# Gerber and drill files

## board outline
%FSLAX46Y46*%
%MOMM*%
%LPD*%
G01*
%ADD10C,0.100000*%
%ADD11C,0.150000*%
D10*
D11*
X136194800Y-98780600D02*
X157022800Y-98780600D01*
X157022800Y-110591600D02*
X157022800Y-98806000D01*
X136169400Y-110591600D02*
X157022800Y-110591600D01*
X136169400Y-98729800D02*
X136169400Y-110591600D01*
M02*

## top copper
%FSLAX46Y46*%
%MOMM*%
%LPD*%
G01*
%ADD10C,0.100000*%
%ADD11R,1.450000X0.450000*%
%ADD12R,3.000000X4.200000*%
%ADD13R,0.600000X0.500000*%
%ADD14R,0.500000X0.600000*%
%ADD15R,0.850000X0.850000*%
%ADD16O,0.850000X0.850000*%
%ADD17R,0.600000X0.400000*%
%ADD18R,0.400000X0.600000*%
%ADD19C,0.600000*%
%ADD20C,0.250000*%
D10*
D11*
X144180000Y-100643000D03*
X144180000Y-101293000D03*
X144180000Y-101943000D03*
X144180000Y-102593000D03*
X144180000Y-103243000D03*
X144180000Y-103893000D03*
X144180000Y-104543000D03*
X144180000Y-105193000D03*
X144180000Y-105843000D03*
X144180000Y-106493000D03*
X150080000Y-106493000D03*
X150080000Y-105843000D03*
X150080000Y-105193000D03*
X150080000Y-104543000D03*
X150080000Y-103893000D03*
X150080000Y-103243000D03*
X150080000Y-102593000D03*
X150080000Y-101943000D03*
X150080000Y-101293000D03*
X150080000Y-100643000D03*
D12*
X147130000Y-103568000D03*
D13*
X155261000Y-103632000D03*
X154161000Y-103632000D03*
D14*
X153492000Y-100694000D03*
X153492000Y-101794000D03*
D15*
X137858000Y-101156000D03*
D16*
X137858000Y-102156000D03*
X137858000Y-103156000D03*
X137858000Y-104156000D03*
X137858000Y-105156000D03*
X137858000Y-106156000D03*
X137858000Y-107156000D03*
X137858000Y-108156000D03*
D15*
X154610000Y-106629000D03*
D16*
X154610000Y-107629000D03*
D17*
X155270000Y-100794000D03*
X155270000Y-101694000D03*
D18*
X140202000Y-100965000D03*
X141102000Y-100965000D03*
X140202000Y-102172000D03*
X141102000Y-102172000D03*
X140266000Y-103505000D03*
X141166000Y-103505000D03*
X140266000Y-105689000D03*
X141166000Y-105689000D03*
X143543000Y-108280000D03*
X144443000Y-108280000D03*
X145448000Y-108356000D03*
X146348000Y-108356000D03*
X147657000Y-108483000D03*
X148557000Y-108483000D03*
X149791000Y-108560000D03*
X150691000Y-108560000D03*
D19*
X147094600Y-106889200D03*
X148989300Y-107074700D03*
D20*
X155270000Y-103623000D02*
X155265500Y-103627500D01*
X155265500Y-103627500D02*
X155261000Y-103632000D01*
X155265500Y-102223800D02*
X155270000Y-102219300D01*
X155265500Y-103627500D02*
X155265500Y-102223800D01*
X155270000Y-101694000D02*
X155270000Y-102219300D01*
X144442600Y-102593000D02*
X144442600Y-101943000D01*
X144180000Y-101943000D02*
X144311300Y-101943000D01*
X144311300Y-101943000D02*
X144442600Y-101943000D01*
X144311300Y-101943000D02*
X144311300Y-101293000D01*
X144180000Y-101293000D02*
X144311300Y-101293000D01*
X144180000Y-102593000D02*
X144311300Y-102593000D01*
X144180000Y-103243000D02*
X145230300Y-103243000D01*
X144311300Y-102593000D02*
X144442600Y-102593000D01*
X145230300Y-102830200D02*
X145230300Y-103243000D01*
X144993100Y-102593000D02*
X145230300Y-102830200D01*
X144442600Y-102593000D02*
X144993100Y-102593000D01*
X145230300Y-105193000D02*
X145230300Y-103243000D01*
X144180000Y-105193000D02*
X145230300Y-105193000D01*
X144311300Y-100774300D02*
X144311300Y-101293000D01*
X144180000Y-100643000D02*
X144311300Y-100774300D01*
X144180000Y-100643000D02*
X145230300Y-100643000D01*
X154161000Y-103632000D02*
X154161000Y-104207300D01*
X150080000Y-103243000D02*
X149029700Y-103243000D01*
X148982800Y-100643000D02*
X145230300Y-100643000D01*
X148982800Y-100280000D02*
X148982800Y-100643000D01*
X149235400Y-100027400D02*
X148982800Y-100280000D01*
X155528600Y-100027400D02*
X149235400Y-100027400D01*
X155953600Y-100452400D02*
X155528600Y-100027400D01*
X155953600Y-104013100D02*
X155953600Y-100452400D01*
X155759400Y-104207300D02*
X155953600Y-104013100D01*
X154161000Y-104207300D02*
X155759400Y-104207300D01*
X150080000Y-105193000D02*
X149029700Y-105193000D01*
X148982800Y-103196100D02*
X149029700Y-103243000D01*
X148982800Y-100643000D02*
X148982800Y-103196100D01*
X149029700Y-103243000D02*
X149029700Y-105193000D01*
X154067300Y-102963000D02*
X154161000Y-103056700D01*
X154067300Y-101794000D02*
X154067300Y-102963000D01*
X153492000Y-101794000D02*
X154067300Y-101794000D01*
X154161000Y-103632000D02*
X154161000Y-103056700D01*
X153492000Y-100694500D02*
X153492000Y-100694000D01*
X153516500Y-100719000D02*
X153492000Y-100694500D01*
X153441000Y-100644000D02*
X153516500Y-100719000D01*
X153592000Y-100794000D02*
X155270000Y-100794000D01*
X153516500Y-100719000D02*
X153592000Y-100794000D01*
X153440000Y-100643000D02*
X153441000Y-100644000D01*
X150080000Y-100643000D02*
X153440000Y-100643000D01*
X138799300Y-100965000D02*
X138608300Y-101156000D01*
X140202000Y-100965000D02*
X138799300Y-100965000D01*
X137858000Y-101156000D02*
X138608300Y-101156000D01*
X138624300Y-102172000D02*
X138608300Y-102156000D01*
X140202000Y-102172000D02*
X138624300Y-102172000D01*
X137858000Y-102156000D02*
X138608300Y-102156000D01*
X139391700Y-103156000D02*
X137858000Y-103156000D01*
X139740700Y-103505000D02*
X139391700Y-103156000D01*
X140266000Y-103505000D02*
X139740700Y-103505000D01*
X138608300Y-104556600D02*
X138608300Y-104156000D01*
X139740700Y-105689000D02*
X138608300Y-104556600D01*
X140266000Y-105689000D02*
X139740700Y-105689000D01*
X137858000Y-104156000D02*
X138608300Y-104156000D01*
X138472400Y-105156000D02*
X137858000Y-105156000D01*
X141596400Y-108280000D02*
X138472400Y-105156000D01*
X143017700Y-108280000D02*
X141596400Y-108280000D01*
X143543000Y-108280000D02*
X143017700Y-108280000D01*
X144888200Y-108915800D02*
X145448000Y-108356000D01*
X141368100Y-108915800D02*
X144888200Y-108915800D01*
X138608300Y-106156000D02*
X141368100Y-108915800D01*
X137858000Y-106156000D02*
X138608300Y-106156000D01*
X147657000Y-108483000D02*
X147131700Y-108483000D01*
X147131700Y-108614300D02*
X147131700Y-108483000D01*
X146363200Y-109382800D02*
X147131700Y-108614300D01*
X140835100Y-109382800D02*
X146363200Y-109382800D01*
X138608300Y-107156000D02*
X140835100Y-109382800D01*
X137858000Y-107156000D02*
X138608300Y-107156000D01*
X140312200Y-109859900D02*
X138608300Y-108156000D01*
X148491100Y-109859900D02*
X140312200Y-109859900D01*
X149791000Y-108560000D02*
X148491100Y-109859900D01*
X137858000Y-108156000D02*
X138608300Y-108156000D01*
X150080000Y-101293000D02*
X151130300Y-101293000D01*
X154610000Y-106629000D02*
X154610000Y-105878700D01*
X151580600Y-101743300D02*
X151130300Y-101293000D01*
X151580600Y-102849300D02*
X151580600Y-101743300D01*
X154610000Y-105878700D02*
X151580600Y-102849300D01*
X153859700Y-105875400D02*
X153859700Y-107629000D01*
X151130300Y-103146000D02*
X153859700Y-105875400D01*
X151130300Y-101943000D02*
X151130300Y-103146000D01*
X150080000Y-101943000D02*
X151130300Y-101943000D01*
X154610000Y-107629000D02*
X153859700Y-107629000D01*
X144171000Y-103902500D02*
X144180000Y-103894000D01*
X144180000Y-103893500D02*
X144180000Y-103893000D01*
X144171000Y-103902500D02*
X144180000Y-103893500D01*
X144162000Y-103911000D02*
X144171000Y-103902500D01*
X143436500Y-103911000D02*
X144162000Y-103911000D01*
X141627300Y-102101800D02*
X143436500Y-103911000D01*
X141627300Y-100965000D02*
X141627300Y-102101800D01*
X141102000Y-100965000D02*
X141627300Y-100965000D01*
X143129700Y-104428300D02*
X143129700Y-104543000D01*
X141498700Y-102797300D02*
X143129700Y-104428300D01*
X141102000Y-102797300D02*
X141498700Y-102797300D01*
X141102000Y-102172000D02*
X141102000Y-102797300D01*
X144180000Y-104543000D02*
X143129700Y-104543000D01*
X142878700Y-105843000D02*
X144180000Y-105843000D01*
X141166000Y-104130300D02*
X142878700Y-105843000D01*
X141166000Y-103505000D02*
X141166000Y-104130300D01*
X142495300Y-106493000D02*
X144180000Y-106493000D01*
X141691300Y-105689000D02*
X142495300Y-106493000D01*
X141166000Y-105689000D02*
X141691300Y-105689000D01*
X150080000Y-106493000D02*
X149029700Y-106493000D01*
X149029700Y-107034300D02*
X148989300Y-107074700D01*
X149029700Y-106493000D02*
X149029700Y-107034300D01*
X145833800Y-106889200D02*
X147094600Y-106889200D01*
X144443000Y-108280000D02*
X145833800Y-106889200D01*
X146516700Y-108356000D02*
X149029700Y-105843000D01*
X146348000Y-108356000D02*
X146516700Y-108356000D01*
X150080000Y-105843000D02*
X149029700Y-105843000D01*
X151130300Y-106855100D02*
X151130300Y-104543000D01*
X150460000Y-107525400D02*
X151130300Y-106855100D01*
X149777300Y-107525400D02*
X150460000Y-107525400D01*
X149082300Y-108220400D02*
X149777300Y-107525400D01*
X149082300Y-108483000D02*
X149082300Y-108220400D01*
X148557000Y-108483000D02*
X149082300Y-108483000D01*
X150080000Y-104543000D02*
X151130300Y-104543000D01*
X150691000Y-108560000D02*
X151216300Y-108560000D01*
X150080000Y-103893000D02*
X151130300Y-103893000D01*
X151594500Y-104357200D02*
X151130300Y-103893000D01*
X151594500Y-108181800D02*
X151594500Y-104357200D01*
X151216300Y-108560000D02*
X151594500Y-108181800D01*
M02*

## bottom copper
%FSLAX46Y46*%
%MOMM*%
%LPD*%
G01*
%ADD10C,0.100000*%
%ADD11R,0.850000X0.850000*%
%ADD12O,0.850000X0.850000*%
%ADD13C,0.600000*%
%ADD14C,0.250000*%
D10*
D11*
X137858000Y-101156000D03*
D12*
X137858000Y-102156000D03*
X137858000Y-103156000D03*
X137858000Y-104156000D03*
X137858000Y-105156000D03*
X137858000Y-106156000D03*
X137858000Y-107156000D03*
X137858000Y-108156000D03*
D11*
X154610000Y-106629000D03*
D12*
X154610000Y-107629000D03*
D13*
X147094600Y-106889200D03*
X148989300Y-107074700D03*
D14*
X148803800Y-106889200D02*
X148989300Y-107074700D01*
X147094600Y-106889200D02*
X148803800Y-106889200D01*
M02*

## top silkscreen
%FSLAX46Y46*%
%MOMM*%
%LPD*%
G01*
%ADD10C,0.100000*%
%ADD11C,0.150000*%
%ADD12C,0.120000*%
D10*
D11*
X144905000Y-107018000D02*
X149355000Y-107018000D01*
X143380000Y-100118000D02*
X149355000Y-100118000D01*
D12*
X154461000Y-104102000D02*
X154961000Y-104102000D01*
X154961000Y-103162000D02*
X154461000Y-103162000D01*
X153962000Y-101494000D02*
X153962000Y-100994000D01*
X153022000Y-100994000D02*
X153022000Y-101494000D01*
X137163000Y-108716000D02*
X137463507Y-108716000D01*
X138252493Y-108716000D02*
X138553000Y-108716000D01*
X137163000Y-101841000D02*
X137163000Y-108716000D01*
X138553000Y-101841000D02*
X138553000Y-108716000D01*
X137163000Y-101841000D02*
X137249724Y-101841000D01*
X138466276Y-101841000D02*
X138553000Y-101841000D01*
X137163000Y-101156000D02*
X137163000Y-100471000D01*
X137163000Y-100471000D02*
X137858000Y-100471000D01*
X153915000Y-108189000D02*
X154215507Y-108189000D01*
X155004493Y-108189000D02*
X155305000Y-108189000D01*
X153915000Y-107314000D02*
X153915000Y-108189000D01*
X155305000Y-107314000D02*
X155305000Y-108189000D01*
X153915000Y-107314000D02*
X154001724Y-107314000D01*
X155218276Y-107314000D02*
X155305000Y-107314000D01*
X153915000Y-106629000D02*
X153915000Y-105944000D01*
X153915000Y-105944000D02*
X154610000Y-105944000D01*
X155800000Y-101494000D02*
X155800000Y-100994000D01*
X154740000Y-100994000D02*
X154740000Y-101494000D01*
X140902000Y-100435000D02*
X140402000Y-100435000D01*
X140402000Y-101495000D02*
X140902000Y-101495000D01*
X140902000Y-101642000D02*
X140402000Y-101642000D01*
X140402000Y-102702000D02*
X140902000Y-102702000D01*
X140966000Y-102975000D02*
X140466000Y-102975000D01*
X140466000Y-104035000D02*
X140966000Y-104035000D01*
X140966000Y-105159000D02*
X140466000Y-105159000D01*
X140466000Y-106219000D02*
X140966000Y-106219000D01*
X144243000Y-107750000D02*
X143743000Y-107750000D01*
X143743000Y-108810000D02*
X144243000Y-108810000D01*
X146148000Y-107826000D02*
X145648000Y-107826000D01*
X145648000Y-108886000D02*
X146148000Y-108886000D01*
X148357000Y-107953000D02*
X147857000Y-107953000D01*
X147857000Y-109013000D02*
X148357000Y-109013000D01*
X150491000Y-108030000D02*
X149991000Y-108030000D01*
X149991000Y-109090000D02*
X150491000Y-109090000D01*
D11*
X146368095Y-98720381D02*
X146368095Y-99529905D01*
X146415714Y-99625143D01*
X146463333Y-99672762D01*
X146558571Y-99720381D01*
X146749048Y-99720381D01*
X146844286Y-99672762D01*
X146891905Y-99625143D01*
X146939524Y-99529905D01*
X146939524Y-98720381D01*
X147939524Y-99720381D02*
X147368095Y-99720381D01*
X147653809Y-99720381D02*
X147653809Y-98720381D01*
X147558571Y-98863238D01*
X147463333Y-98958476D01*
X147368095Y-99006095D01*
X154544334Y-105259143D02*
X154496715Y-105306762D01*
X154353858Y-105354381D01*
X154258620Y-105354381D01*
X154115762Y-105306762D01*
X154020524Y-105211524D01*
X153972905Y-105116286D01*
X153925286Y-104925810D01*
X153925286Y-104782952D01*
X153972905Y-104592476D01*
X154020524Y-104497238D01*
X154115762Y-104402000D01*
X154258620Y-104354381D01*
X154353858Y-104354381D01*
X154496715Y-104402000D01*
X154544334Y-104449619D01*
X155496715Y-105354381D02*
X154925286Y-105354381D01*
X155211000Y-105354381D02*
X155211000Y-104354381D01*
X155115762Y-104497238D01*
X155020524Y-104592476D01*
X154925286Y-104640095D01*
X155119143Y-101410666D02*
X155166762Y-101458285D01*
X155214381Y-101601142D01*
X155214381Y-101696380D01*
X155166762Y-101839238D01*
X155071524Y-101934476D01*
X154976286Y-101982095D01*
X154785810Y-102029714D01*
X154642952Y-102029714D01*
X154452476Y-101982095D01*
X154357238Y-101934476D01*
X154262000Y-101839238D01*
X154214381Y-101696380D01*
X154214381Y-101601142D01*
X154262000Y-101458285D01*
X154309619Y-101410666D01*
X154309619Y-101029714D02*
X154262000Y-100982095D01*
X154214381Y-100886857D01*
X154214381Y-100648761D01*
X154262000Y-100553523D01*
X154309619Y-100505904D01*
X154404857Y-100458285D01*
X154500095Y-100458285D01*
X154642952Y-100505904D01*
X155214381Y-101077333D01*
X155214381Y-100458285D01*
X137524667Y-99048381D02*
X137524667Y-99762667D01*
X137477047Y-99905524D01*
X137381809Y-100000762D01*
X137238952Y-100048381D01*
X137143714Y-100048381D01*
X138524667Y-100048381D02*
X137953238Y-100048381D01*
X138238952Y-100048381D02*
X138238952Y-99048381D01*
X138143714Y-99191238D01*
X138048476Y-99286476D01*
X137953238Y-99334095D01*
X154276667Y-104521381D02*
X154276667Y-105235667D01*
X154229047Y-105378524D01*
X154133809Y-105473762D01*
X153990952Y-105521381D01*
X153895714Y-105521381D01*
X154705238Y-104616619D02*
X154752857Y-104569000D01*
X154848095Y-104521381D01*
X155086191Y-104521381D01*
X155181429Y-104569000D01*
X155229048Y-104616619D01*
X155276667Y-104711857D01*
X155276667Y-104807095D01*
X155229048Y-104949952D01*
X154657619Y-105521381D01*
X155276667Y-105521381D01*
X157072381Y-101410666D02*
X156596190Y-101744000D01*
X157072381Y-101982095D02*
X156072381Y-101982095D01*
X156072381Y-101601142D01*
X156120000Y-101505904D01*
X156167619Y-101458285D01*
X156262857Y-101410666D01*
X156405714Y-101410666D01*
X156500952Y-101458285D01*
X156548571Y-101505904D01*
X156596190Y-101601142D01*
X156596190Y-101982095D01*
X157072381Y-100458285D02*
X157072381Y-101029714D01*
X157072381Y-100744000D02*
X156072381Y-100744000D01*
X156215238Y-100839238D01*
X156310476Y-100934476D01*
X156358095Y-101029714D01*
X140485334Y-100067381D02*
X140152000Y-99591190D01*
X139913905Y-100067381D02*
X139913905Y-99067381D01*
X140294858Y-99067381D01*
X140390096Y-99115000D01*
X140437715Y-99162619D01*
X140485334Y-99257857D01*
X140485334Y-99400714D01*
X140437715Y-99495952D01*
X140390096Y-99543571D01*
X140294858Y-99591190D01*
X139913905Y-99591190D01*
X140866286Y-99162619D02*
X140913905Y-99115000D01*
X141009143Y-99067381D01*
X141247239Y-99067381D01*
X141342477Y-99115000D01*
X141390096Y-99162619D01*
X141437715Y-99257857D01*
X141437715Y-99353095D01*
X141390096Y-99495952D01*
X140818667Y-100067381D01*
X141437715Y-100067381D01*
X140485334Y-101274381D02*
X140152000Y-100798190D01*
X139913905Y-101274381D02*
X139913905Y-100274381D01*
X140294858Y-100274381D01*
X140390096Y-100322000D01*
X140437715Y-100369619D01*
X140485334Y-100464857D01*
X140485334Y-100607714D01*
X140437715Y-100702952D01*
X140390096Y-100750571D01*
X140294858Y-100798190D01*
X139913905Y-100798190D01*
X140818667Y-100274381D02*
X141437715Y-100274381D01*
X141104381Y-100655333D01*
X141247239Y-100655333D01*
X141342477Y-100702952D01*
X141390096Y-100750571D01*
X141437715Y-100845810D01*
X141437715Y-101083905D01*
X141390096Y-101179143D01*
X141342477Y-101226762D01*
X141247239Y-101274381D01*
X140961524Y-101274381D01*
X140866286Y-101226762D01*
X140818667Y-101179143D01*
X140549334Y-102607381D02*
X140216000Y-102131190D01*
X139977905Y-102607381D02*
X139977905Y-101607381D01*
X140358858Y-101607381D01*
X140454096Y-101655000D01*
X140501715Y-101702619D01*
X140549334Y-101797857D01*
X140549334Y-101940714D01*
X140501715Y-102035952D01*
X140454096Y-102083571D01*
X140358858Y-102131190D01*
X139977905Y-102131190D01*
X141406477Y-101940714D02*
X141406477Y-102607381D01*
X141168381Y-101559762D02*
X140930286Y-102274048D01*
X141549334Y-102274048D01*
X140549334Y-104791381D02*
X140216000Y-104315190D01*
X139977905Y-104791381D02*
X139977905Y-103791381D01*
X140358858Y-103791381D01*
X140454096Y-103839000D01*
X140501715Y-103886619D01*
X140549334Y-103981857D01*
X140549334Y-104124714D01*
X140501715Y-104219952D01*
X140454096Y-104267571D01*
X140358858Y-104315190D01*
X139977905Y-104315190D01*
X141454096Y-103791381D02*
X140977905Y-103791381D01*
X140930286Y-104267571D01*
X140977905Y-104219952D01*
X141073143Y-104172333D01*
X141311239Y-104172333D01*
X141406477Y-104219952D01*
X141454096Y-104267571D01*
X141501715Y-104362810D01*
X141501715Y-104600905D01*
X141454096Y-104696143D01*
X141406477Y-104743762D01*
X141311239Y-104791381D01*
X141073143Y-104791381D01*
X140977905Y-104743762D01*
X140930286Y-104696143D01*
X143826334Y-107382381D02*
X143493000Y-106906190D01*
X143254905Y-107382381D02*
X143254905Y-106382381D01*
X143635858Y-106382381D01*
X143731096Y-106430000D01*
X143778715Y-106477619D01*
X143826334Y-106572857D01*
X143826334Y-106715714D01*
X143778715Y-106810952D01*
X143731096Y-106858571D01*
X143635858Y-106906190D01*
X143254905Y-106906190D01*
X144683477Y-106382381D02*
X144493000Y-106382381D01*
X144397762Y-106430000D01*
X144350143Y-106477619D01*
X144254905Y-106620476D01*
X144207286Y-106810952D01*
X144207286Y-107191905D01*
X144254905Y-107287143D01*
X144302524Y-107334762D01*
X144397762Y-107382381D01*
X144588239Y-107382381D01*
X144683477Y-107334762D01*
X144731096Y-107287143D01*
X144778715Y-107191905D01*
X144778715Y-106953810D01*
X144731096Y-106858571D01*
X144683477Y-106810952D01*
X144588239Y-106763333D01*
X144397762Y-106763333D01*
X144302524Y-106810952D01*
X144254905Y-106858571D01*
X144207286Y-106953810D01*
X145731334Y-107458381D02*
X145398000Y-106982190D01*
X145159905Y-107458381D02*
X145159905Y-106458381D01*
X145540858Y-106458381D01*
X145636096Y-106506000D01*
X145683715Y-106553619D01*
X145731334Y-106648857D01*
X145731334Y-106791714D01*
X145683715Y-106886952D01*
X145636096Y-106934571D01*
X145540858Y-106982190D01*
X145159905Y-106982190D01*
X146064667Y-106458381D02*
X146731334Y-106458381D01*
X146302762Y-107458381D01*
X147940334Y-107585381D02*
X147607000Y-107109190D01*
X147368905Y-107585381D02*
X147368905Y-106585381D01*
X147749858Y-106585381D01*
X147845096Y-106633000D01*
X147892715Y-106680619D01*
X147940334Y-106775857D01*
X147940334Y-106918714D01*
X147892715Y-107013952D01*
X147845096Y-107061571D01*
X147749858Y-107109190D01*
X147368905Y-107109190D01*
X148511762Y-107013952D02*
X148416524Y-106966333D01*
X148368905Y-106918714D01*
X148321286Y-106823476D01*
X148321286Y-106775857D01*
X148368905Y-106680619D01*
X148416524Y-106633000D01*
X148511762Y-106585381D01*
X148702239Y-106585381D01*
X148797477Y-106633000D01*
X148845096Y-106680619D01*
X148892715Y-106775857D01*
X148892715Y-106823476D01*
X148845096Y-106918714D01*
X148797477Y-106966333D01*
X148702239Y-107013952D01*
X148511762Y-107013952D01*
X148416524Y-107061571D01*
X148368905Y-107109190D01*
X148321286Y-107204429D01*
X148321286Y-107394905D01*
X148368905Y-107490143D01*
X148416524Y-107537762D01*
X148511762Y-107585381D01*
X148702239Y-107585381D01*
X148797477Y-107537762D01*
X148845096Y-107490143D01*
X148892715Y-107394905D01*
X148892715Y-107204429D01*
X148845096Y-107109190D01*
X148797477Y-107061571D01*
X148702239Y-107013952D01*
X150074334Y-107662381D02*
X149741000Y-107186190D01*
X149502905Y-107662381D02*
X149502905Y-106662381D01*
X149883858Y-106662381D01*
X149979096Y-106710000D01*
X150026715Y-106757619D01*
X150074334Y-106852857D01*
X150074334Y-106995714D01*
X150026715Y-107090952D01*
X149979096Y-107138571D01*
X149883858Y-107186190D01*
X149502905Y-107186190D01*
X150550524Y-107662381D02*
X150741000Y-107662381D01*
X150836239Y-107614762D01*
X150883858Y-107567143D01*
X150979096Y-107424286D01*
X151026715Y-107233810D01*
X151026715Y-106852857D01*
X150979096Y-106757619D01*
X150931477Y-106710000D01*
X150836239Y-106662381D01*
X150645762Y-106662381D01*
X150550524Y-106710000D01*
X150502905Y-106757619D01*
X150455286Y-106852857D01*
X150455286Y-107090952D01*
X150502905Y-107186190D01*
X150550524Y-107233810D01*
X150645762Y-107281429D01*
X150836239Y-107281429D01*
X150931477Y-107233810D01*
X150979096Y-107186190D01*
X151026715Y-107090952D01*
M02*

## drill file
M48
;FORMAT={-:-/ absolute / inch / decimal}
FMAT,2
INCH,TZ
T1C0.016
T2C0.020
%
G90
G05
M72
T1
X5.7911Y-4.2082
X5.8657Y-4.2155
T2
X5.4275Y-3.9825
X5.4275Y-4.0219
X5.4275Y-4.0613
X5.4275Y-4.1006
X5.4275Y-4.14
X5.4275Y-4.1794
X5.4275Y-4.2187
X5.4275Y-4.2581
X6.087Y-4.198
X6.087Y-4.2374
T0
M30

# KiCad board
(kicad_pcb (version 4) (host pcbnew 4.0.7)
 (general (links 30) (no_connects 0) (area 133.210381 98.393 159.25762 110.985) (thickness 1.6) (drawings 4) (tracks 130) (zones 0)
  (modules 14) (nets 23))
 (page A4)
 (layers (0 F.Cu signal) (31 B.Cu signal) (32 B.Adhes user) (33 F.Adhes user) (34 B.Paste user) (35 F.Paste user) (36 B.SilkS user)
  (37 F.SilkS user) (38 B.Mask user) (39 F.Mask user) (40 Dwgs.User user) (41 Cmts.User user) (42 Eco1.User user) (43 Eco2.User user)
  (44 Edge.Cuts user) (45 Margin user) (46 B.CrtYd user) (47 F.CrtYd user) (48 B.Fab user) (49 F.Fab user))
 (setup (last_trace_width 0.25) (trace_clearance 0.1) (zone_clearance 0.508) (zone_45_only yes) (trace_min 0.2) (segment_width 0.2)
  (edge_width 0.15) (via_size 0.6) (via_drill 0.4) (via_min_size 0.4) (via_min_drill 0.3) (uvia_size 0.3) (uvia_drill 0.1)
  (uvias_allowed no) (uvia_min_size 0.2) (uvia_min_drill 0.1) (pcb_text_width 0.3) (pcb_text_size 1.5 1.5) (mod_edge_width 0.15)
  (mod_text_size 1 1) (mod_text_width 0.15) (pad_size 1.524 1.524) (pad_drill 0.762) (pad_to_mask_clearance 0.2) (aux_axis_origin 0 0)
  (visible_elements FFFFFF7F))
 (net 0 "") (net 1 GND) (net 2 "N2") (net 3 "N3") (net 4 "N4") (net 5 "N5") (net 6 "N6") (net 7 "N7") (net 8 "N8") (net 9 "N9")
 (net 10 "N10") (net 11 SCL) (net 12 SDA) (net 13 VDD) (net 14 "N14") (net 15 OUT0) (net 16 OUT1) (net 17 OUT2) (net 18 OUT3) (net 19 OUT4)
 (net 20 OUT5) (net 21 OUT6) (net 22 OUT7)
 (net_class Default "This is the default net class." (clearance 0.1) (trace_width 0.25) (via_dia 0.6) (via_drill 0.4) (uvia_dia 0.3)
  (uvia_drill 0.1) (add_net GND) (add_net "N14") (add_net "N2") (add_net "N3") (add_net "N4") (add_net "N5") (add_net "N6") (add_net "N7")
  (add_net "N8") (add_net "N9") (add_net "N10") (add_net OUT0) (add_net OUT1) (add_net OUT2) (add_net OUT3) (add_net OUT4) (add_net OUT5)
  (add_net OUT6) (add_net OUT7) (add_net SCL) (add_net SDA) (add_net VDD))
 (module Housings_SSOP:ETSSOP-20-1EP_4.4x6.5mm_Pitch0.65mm (layer F.Cu) (at 147.13 103.568)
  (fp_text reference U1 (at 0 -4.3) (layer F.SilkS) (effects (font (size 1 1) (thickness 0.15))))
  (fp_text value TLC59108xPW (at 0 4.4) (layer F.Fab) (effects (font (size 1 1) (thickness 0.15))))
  (fp_line (start -2.225 3.45) (end 2.225 3.45) (layer F.SilkS) (width 0.15))
  (fp_line (start -3.75 -3.45) (end 2.225 -3.45) (layer F.SilkS) (width 0.15))
  (pad 1 smd rect (at -2.95 -2.925) (size 1.45 0.45) (layers F.Cu F.Paste F.Mask) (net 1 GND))
  (pad 2 smd rect (at -2.95 -2.275) (size 1.45 0.45) (layers F.Cu F.Paste F.Mask) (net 1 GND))
  (pad 3 smd rect (at -2.95 -1.625) (size 1.45 0.45) (layers F.Cu F.Paste F.Mask) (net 1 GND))
  (pad 4 smd rect (at -2.95 -0.975) (size 1.45 0.45) (layers F.Cu F.Paste F.Mask) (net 1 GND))
  (pad 5 smd rect (at -2.95 -0.325) (size 1.45 0.45) (layers F.Cu F.Paste F.Mask) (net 1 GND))
  (pad 6 smd rect (at -2.95 0.325) (size 1.45 0.45) (layers F.Cu F.Paste F.Mask) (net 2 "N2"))
  (pad 7 smd rect (at -2.95 0.975) (size 1.45 0.45) (layers F.Cu F.Paste F.Mask) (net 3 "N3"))
  (pad 8 smd rect (at -2.95 1.625) (size 1.45 0.45) (layers F.Cu F.Paste F.Mask) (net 1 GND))
  (pad 9 smd rect (at -2.95 2.275) (size 1.45 0.45) (layers F.Cu F.Paste F.Mask) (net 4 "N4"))
  (pad 10 smd rect (at -2.95 2.925) (size 1.45 0.45) (layers F.Cu F.Paste F.Mask) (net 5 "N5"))
  (pad 11 smd rect (at 2.95 2.925) (size 1.45 0.45) (layers F.Cu F.Paste F.Mask) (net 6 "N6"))
  (pad 12 smd rect (at 2.95 2.275) (size 1.45 0.45) (layers F.Cu F.Paste F.Mask) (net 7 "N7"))
  (pad 13 smd rect (at 2.95 1.625) (size 1.45 0.45) (layers F.Cu F.Paste F.Mask) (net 1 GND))
  (pad 14 smd rect (at 2.95 0.975) (size 1.45 0.45) (layers F.Cu F.Paste F.Mask) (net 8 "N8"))
  (pad 15 smd rect (at 2.95 0.325) (size 1.45 0.45) (layers F.Cu F.Paste F.Mask) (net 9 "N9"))
  (pad 16 smd rect (at 2.95 -0.325) (size 1.45 0.45) (layers F.Cu F.Paste F.Mask) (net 1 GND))
  (pad 17 smd rect (at 2.95 -0.975) (size 1.45 0.45) (layers F.Cu F.Paste F.Mask) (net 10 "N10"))
  (pad 18 smd rect (at 2.95 -1.625) (size 1.45 0.45) (layers F.Cu F.Paste F.Mask) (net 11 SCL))
  (pad 19 smd rect (at 2.95 -2.275) (size 1.45 0.45) (layers F.Cu F.Paste F.Mask) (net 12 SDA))
  (pad 20 smd rect (at 2.95 -2.925) (size 1.45 0.45) (layers F.Cu F.Paste F.Mask) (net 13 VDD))
  (pad 21 smd rect (at 0 0) (size 3 4.2) (layers F.Cu F.Paste F.Mask)))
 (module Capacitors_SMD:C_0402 (layer F.Cu) (at 154.711 103.632 180)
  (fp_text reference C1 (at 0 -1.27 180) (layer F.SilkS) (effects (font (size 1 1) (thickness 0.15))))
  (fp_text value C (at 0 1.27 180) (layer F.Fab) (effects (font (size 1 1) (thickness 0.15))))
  (fp_line (start 0.25 -0.47) (end -0.25 -0.47) (layer F.SilkS) (width 0.12))
  (fp_line (start -0.25 0.47) (end 0.25 0.47) (layer F.SilkS) (width 0.12))
  (pad 1 smd rect (at -0.55 0 180) (size 0.6 0.5) (layers F.Cu F.Paste F.Mask) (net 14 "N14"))
  (pad 2 smd rect (at 0.55 0 180) (size 0.6 0.5) (layers F.Cu F.Paste F.Mask) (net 1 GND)))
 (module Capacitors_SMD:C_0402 (layer F.Cu) (at 153.492 101.244 270)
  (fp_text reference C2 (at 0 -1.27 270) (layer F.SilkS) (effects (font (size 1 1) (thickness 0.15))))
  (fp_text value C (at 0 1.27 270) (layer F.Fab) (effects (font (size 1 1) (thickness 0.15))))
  (fp_line (start 0.25 -0.47) (end -0.25 -0.47) (layer F.SilkS) (width 0.12))
  (fp_line (start -0.25 0.47) (end 0.25 0.47) (layer F.SilkS) (width 0.12))
  (pad 1 smd rect (at -0.55 0 270) (size 0.6 0.5) (layers F.Cu F.Paste F.Mask) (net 13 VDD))
  (pad 2 smd rect (at 0.55 0 270) (size 0.6 0.5) (layers F.Cu F.Paste F.Mask) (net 1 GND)))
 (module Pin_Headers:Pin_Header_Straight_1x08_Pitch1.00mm (layer F.Cu) (at 137.858 101.156)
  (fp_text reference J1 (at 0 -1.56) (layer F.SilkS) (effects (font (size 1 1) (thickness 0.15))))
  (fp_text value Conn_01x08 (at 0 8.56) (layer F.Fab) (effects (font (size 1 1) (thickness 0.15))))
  (fp_line (start -0.695 7.56) (end -0.394493 7.56) (layer F.SilkS) (width 0.12))
  (fp_line (start 0.394493 7.56) (end 0.695 7.56) (layer F.SilkS) (width 0.12))
  (fp_line (start -0.695 0.685) (end -0.695 7.56) (layer F.SilkS) (width 0.12))
  (fp_line (start 0.695 0.685) (end 0.695 7.56) (layer F.SilkS) (width 0.12))
  (fp_line (start -0.695 0.685) (end -0.608276 0.685) (layer F.SilkS) (width 0.12))
  (fp_line (start 0.608276 0.685) (end 0.695 0.685) (layer F.SilkS) (width 0.12))
  (fp_line (start -0.695 0) (end -0.695 -0.685) (layer F.SilkS) (width 0.12))
  (fp_line (start -0.695 -0.685) (end 0 -0.685) (layer F.SilkS) (width 0.12))
  (pad 1 thru_hole rect (at 0 0) (size 0.85 0.85) (drill 0.5) (layers *.Cu *.Mask) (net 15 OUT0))
  (pad 2 thru_hole oval (at 0 1) (size 0.85 0.85) (drill 0.5) (layers *.Cu *.Mask) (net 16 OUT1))
  (pad 3 thru_hole oval (at 0 2) (size 0.85 0.85) (drill 0.5) (layers *.Cu *.Mask) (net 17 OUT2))
  (pad 4 thru_hole oval (at 0 3) (size 0.85 0.85) (drill 0.5) (layers *.Cu *.Mask) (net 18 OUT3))
  (pad 5 thru_hole oval (at 0 4) (size 0.85 0.85) (drill 0.5) (layers *.Cu *.Mask) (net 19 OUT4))
  (pad 6 thru_hole oval (at 0 5) (size 0.85 0.85) (drill 0.5) (layers *.Cu *.Mask) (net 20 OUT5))
  (pad 7 thru_hole oval (at 0 6) (size 0.85 0.85) (drill 0.5) (layers *.Cu *.Mask) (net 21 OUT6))
  (pad 8 thru_hole oval (at 0 7) (size 0.85 0.85) (drill 0.5) (layers *.Cu *.Mask) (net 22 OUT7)))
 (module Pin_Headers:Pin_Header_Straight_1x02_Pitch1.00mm (layer F.Cu) (at 154.61 106.629)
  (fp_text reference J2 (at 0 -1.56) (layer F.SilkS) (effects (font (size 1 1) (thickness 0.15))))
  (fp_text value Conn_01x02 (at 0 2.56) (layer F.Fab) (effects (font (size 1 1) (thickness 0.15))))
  (fp_line (start -0.695 1.56) (end -0.394493 1.56) (layer F.SilkS) (width 0.12))
  (fp_line (start 0.394493 1.56) (end 0.695 1.56) (layer F.SilkS) (width 0.12))
  (fp_line (start -0.695 0.685) (end -0.695 1.56) (layer F.SilkS) (width 0.12))
  (fp_line (start 0.695 0.685) (end 0.695 1.56) (layer F.SilkS) (width 0.12))
  (fp_line (start -0.695 0.685) (end -0.608276 0.685) (layer F.SilkS) (width 0.12))
  (fp_line (start 0.608276 0.685) (end 0.695 0.685) (layer F.SilkS) (width 0.12))
  (fp_line (start -0.695 0) (end -0.695 -0.685) (layer F.SilkS) (width 0.12))
  (fp_line (start -0.695 -0.685) (end 0 -0.685) (layer F.SilkS) (width 0.12))
  (pad 1 thru_hole rect (at 0 0) (size 0.85 0.85) (drill 0.5) (layers *.Cu *.Mask) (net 12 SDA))
  (pad 2 thru_hole oval (at 0 1) (size 0.85 0.85) (drill 0.5) (layers *.Cu *.Mask) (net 11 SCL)))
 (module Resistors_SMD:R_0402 (layer F.Cu) (at 155.27 101.244 270)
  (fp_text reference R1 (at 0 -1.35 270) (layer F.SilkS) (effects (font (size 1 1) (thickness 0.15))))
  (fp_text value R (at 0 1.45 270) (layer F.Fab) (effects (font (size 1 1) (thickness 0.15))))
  (fp_line (start 0.25 -0.53) (end -0.25 -0.53) (layer F.SilkS) (width 0.12))
  (fp_line (start -0.25 0.53) (end 0.25 0.53) (layer F.SilkS) (width 0.12))
  (pad 1 smd rect (at -0.45 0 270) (size 0.4 0.6) (layers F.Cu F.Paste F.Mask) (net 13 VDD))
  (pad 2 smd rect (at 0.45 0 270) (size 0.4 0.6) (layers F.Cu F.Paste F.Mask) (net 14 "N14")))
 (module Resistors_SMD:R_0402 (layer F.Cu) (at 140.652 100.965)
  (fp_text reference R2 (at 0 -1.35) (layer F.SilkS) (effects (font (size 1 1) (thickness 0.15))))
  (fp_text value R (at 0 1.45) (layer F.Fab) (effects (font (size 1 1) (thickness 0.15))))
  (fp_line (start 0.25 -0.53) (end -0.25 -0.53) (layer F.SilkS) (width 0.12))
  (fp_line (start -0.25 0.53) (end 0.25 0.53) (layer F.SilkS) (width 0.12))
  (pad 1 smd rect (at -0.45 0) (size 0.4 0.6) (layers F.Cu F.Paste F.Mask) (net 15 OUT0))
  (pad 2 smd rect (at 0.45 0) (size 0.4 0.6) (layers F.Cu F.Paste F.Mask) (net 2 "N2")))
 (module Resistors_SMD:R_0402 (layer F.Cu) (at 140.652 102.172)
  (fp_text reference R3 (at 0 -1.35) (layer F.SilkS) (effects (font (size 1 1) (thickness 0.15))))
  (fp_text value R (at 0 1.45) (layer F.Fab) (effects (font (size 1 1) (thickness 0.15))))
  (fp_line (start 0.25 -0.53) (end -0.25 -0.53) (layer F.SilkS) (width 0.12))
  (fp_line (start -0.25 0.53) (end 0.25 0.53) (layer F.SilkS) (width 0.12))
  (pad 1 smd rect (at -0.45 0) (size 0.4 0.6) (layers F.Cu F.Paste F.Mask) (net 16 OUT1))
  (pad 2 smd rect (at 0.45 0) (size 0.4 0.6) (layers F.Cu F.Paste F.Mask) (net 3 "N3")))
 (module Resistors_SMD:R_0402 (layer F.Cu) (at 140.716 103.505)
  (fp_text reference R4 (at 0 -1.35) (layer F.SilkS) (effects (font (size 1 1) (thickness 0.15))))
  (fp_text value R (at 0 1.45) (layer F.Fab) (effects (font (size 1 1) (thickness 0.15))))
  (fp_line (start 0.25 -0.53) (end -0.25 -0.53) (layer F.SilkS) (width 0.12))
  (fp_line (start -0.25 0.53) (end 0.25 0.53) (layer F.SilkS) (width 0.12))
  (pad 1 smd rect (at -0.45 0) (size 0.4 0.6) (layers F.Cu F.Paste F.Mask) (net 17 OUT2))
  (pad 2 smd rect (at 0.45 0) (size 0.4 0.6) (layers F.Cu F.Paste F.Mask) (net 4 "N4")))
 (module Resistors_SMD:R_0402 (layer F.Cu) (at 140.716 105.689)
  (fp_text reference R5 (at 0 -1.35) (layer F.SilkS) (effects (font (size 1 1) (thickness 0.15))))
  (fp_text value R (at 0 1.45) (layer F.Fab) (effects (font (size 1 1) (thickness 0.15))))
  (fp_line (start 0.25 -0.53) (end -0.25 -0.53) (layer F.SilkS) (width 0.12))
  (fp_line (start -0.25 0.53) (end 0.25 0.53) (layer F.SilkS) (width 0.12))
  (pad 1 smd rect (at -0.45 0) (size 0.4 0.6) (layers F.Cu F.Paste F.Mask) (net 18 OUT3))
  (pad 2 smd rect (at 0.45 0) (size 0.4 0.6) (layers F.Cu F.Paste F.Mask) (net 5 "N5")))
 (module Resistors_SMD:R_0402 (layer F.Cu) (at 143.993 108.28)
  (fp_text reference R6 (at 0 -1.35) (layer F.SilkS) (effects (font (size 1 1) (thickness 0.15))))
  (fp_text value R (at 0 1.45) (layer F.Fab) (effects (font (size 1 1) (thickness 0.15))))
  (fp_line (start 0.25 -0.53) (end -0.25 -0.53) (layer F.SilkS) (width 0.12))
  (fp_line (start -0.25 0.53) (end 0.25 0.53) (layer F.SilkS) (width 0.12))
  (pad 1 smd rect (at -0.45 0) (size 0.4 0.6) (layers F.Cu F.Paste F.Mask) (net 19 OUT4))
  (pad 2 smd rect (at 0.45 0) (size 0.4 0.6) (layers F.Cu F.Paste F.Mask) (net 6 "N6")))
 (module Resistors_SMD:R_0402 (layer F.Cu) (at 145.898 108.356)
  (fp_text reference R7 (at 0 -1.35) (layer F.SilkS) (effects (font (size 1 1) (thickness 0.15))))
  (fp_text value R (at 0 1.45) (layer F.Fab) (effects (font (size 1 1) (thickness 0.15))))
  (fp_line (start 0.25 -0.53) (end -0.25 -0.53) (layer F.SilkS) (width 0.12))
  (fp_line (start -0.25 0.53) (end 0.25 0.53) (layer F.SilkS) (width 0.12))
  (pad 1 smd rect (at -0.45 0) (size 0.4 0.6) (layers F.Cu F.Paste F.Mask) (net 20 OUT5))
  (pad 2 smd rect (at 0.45 0) (size 0.4 0.6) (layers F.Cu F.Paste F.Mask) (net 7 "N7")))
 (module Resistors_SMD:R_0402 (layer F.Cu) (at 148.107 108.483)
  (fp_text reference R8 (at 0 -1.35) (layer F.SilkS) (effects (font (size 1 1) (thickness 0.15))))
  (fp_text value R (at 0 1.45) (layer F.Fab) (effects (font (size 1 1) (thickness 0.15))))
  (fp_line (start 0.25 -0.53) (end -0.25 -0.53) (layer F.SilkS) (width 0.12))
  (fp_line (start -0.25 0.53) (end 0.25 0.53) (layer F.SilkS) (width 0.12))
  (pad 1 smd rect (at -0.45 0) (size 0.4 0.6) (layers F.Cu F.Paste F.Mask) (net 21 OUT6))
  (pad 2 smd rect (at 0.45 0) (size 0.4 0.6) (layers F.Cu F.Paste F.Mask) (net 8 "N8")))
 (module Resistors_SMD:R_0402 (layer F.Cu) (at 150.241 108.56)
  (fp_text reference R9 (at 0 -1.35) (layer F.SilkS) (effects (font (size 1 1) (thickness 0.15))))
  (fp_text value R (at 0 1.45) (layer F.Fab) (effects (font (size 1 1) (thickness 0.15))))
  (fp_line (start 0.25 -0.53) (end -0.25 -0.53) (layer F.SilkS) (width 0.12))
  (fp_line (start -0.25 0.53) (end 0.25 0.53) (layer F.SilkS) (width 0.12))
  (pad 1 smd rect (at -0.45 0) (size 0.4 0.6) (layers F.Cu F.Paste F.Mask) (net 22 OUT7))
  (pad 2 smd rect (at 0.45 0) (size 0.4 0.6) (layers F.Cu F.Paste F.Mask) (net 9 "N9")))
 (gr_line (start 136.1948 98.7806) (end 157.0228 98.7806) (angle 90) (layer Edge.Cuts) (width 0.15))
 (gr_line (start 157.0228 110.5916) (end 157.0228 98.806) (angle 90) (layer Edge.Cuts) (width 0.15))
 (gr_line (start 136.1694 110.5916) (end 157.0228 110.5916) (angle 90) (layer Edge.Cuts) (width 0.15))
 (gr_line (start 136.1694 98.7298) (end 136.1694 110.5916) (angle 90) (layer Edge.Cuts) (width 0.15))
 (segment (start 155.27 103.623) (end 155.2655 103.6275) (width 0.25) (layer F.Cu) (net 14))
 (segment (start 155.2655 103.6275) (end 155.261 103.632) (width 0.25) (layer F.Cu) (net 14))
 (segment (start 155.2655 102.2238) (end 155.27 102.2193) (width 0.25) (layer F.Cu) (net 14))
 (segment (start 155.2655 103.6275) (end 155.2655 102.2238) (width 0.25) (layer F.Cu) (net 14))
 (segment (start 155.27 101.694) (end 155.27 102.2193) (width 0.25) (layer F.Cu) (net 14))
 (segment (start 144.4426 102.593) (end 144.4426 101.943) (width 0.25) (layer F.Cu) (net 1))
 (segment (start 144.18 101.943) (end 144.3113 101.943) (width 0.25) (layer F.Cu) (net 1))
 (segment (start 144.3113 101.943) (end 144.4426 101.943) (width 0.25) (layer F.Cu) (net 1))
 (segment (start 144.3113 101.943) (end 144.3113 101.293) (width 0.25) (layer F.Cu) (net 1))
 (segment (start 144.18 101.293) (end 144.3113 101.293) (width 0.25) (layer F.Cu) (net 1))
 (segment (start 144.18 102.593) (end 144.3113 102.593) (width 0.25) (layer F.Cu) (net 1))
 (segment (start 144.18 103.243) (end 145.2303 103.243) (width 0.25) (layer F.Cu) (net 1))
 (segment (start 144.3113 102.593) (end 144.4426 102.593) (width 0.25) (layer F.Cu) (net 1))
 (segment (start 145.2303 102.8302) (end 145.2303 103.243) (width 0.25) (layer F.Cu) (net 1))
 (segment (start 144.9931 102.593) (end 145.2303 102.8302) (width 0.25) (layer F.Cu) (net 1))
 (segment (start 144.4426 102.593) (end 144.9931 102.593) (width 0.25) (layer F.Cu) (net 1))
 (segment (start 145.2303 105.193) (end 145.2303 103.243) (width 0.25) (layer F.Cu) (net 1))
 (segment (start 144.18 105.193) (end 145.2303 105.193) (width 0.25) (layer F.Cu) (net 1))
 (segment (start 144.3113 100.7743) (end 144.3113 101.293) (width 0.25) (layer F.Cu) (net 1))
 (segment (start 144.18 100.643) (end 144.3113 100.7743) (width 0.25) (layer F.Cu) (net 1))
 (segment (start 144.18 100.643) (end 145.2303 100.643) (width 0.25) (layer F.Cu) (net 1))
 (segment (start 154.161 103.632) (end 154.161 104.2073) (width 0.25) (layer F.Cu) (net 1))
 (segment (start 150.08 103.243) (end 149.0297 103.243) (width 0.25) (layer F.Cu) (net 1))
 (segment (start 148.9828 100.643) (end 145.2303 100.643) (width 0.25) (layer F.Cu) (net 1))
 (segment (start 148.9828 100.28) (end 148.9828 100.643) (width 0.25) (layer F.Cu) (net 1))
 (segment (start 149.2354 100.0274) (end 148.9828 100.28) (width 0.25) (layer F.Cu) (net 1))
 (segment (start 155.5286 100.0274) (end 149.2354 100.0274) (width 0.25) (layer F.Cu) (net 1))
 (segment (start 155.9536 100.4524) (end 155.5286 100.0274) (width 0.25) (layer F.Cu) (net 1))
 (segment (start 155.9536 104.0131) (end 155.9536 100.4524) (width 0.25) (layer F.Cu) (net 1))
 (segment (start 155.7594 104.2073) (end 155.9536 104.0131) (width 0.25) (layer F.Cu) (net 1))
 (segment (start 154.161 104.2073) (end 155.7594 104.2073) (width 0.25) (layer F.Cu) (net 1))
 (segment (start 150.08 105.193) (end 149.0297 105.193) (width 0.25) (layer F.Cu) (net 1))
 (segment (start 148.9828 103.1961) (end 149.0297 103.243) (width 0.25) (layer F.Cu) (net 1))
 (segment (start 148.9828 100.643) (end 148.9828 103.1961) (width 0.25) (layer F.Cu) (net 1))
 (segment (start 149.0297 103.243) (end 149.0297 105.193) (width 0.25) (layer F.Cu) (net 1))
 (segment (start 154.0673 102.963) (end 154.161 103.0567) (width 0.25) (layer F.Cu) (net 1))
 (segment (start 154.0673 101.794) (end 154.0673 102.963) (width 0.25) (layer F.Cu) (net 1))
 (segment (start 153.492 101.794) (end 154.0673 101.794) (width 0.25) (layer F.Cu) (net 1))
 (segment (start 154.161 103.632) (end 154.161 103.0567) (width 0.25) (layer F.Cu) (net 1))
 (segment (start 153.492 100.6945) (end 153.492 100.694) (width 0.25) (layer F.Cu) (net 13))
 (segment (start 153.5165 100.719) (end 153.492 100.6945) (width 0.25) (layer F.Cu) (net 13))
 (segment (start 153.441 100.644) (end 153.5165 100.719) (width 0.25) (layer F.Cu) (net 13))
 (segment (start 153.592 100.794) (end 155.27 100.794) (width 0.25) (layer F.Cu) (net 13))
 (segment (start 153.5165 100.719) (end 153.592 100.794) (width 0.25) (layer F.Cu) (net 13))
 (segment (start 153.44 100.643) (end 153.441 100.644) (width 0.25) (layer F.Cu) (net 13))
 (segment (start 150.08 100.643) (end 153.44 100.643) (width 0.25) (layer F.Cu) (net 13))
 (segment (start 138.7993 100.965) (end 138.6083 101.156) (width 0.25) (layer F.Cu) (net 15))
 (segment (start 140.202 100.965) (end 138.7993 100.965) (width 0.25) (layer F.Cu) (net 15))
 (segment (start 137.858 101.156) (end 138.6083 101.156) (width 0.25) (layer F.Cu) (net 15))
 (segment (start 138.6243 102.172) (end 138.6083 102.156) (width 0.25) (layer F.Cu) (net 16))
 (segment (start 140.202 102.172) (end 138.6243 102.172) (width 0.25) (layer F.Cu) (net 16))
 (segment (start 137.858 102.156) (end 138.6083 102.156) (width 0.25) (layer F.Cu) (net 16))
 (segment (start 139.3917 103.156) (end 137.858 103.156) (width 0.25) (layer F.Cu) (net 17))
 (segment (start 139.7407 103.505) (end 139.3917 103.156) (width 0.25) (layer F.Cu) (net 17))
 (segment (start 140.266 103.505) (end 139.7407 103.505) (width 0.25) (layer F.Cu) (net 17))
 (segment (start 138.6083 104.5566) (end 138.6083 104.156) (width 0.25) (layer F.Cu) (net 18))
 (segment (start 139.7407 105.689) (end 138.6083 104.5566) (width 0.25) (layer F.Cu) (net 18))
 (segment (start 140.266 105.689) (end 139.7407 105.689) (width 0.25) (layer F.Cu) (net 18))
 (segment (start 137.858 104.156) (end 138.6083 104.156) (width 0.25) (layer F.Cu) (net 18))
 (segment (start 138.4724 105.156) (end 137.858 105.156) (width 0.25) (layer F.Cu) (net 19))
 (segment (start 141.5964 108.28) (end 138.4724 105.156) (width 0.25) (layer F.Cu) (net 19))
 (segment (start 143.0177 108.28) (end 141.5964 108.28) (width 0.25) (layer F.Cu) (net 19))
 (segment (start 143.543 108.28) (end 143.0177 108.28) (width 0.25) (layer F.Cu) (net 19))
 (segment (start 144.8882 108.9158) (end 145.448 108.356) (width 0.25) (layer F.Cu) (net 20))
 (segment (start 141.3681 108.9158) (end 144.8882 108.9158) (width 0.25) (layer F.Cu) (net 20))
 (segment (start 138.6083 106.156) (end 141.3681 108.9158) (width 0.25) (layer F.Cu) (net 20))
 (segment (start 137.858 106.156) (end 138.6083 106.156) (width 0.25) (layer F.Cu) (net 20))
 (segment (start 147.657 108.483) (end 147.1317 108.483) (width 0.25) (layer F.Cu) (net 21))
 (segment (start 147.1317 108.6143) (end 147.1317 108.483) (width 0.25) (layer F.Cu) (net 21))
 (segment (start 146.3632 109.3828) (end 147.1317 108.6143) (width 0.25) (layer F.Cu) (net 21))
 (segment (start 140.8351 109.3828) (end 146.3632 109.3828) (width 0.25) (layer F.Cu) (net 21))
 (segment (start 138.6083 107.156) (end 140.8351 109.3828) (width 0.25) (layer F.Cu) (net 21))
 (segment (start 137.858 107.156) (end 138.6083 107.156) (width 0.25) (layer F.Cu) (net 21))
 (segment (start 140.3122 109.8599) (end 138.6083 108.156) (width 0.25) (layer F.Cu) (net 22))
 (segment (start 148.4911 109.8599) (end 140.3122 109.8599) (width 0.25) (layer F.Cu) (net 22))
 (segment (start 149.791 108.56) (end 148.4911 109.8599) (width 0.25) (layer F.Cu) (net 22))
 (segment (start 137.858 108.156) (end 138.6083 108.156) (width 0.25) (layer F.Cu) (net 22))
 (segment (start 150.08 101.293) (end 151.1303 101.293) (width 0.25) (layer F.Cu) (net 12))
 (segment (start 154.61 106.629) (end 154.61 105.8787) (width 0.25) (layer F.Cu) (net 12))
 (segment (start 151.5806 101.7433) (end 151.1303 101.293) (width 0.25) (layer F.Cu) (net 12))
 (segment (start 151.5806 102.8493) (end 151.5806 101.7433) (width 0.25) (layer F.Cu) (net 12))
 (segment (start 154.61 105.8787) (end 151.5806 102.8493) (width 0.25) (layer F.Cu) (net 12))
 (segment (start 153.8597 105.8754) (end 153.8597 107.629) (width 0.25) (layer F.Cu) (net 11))
 (segment (start 151.1303 103.146) (end 153.8597 105.8754) (width 0.25) (layer F.Cu) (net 11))
 (segment (start 151.1303 101.943) (end 151.1303 103.146) (width 0.25) (layer F.Cu) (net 11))
 (segment (start 150.08 101.943) (end 151.1303 101.943) (width 0.25) (layer F.Cu) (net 11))
 (segment (start 154.61 107.629) (end 153.8597 107.629) (width 0.25) (layer F.Cu) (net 11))
 (segment (start 144.171 103.9025) (end 144.18 103.894) (width 0.25) (layer F.Cu) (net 2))
 (segment (start 144.18 103.8935) (end 144.18 103.893) (width 0.25) (layer F.Cu) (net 2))
 (segment (start 144.171 103.9025) (end 144.18 103.8935) (width 0.25) (layer F.Cu) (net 2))
 (segment (start 144.162 103.911) (end 144.171 103.9025) (width 0.25) (layer F.Cu) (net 2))
 (segment (start 143.4365 103.911) (end 144.162 103.911) (width 0.25) (layer F.Cu) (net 2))
 (segment (start 141.6273 102.1018) (end 143.4365 103.911) (width 0.25) (layer F.Cu) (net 2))
 (segment (start 141.6273 100.965) (end 141.6273 102.1018) (width 0.25) (layer F.Cu) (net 2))
 (segment (start 141.102 100.965) (end 141.6273 100.965) (width 0.25) (layer F.Cu) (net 2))
 (segment (start 143.1297 104.4283) (end 143.1297 104.543) (width 0.25) (layer F.Cu) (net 3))
 (segment (start 141.4987 102.7973) (end 143.1297 104.4283) (width 0.25) (layer F.Cu) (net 3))
 (segment (start 141.102 102.7973) (end 141.4987 102.7973) (width 0.25) (layer F.Cu) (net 3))
 (segment (start 141.102 102.172) (end 141.102 102.7973) (width 0.25) (layer F.Cu) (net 3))
 (segment (start 144.18 104.543) (end 143.1297 104.543) (width 0.25) (layer F.Cu) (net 3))
 (segment (start 142.8787 105.843) (end 144.18 105.843) (width 0.25) (layer F.Cu) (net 4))
 (segment (start 141.166 104.1303) (end 142.8787 105.843) (width 0.25) (layer F.Cu) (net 4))
 (segment (start 141.166 103.505) (end 141.166 104.1303) (width 0.25) (layer F.Cu) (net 4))
 (segment (start 142.4953 106.493) (end 144.18 106.493) (width 0.25) (layer F.Cu) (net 5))
 (segment (start 141.6913 105.689) (end 142.4953 106.493) (width 0.25) (layer F.Cu) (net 5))
 (segment (start 141.166 105.689) (end 141.6913 105.689) (width 0.25) (layer F.Cu) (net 5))
 (via (at 147.0946 106.8892) (size 0.6) (layers F.Cu B.Cu) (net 6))
 (via (at 148.9893 107.0747) (size 0.6) (layers F.Cu B.Cu) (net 6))
 (segment (start 150.08 106.493) (end 149.0297 106.493) (width 0.25) (layer F.Cu) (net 6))
 (segment (start 149.0297 107.0343) (end 148.9893 107.0747) (width 0.25) (layer F.Cu) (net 6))
 (segment (start 149.0297 106.493) (end 149.0297 107.0343) (width 0.25) (layer F.Cu) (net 6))
 (segment (start 148.8038 106.8892) (end 148.9893 107.0747) (width 0.25) (layer B.Cu) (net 6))
 (segment (start 147.0946 106.8892) (end 148.8038 106.8892) (width 0.25) (layer B.Cu) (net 6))
 (segment (start 145.8338 106.8892) (end 147.0946 106.8892) (width 0.25) (layer F.Cu) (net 6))
 (segment (start 144.443 108.28) (end 145.8338 106.8892) (width 0.25) (layer F.Cu) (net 6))
 (segment (start 146.5167 108.356) (end 149.0297 105.843) (width 0.25) (layer F.Cu) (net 7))
 (segment (start 146.348 108.356) (end 146.5167 108.356) (width 0.25) (layer F.Cu) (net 7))
 (segment (start 150.08 105.843) (end 149.0297 105.843) (width 0.25) (layer F.Cu) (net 7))
 (segment (start 151.1303 106.8551) (end 151.1303 104.543) (width 0.25) (layer F.Cu) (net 8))
 (segment (start 150.46 107.5254) (end 151.1303 106.8551) (width 0.25) (layer F.Cu) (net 8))
 (segment (start 149.7773 107.5254) (end 150.46 107.5254) (width 0.25) (layer F.Cu) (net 8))
 (segment (start 149.0823 108.2204) (end 149.7773 107.5254) (width 0.25) (layer F.Cu) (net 8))
 (segment (start 149.0823 108.483) (end 149.0823 108.2204) (width 0.25) (layer F.Cu) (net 8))
 (segment (start 148.557 108.483) (end 149.0823 108.483) (width 0.25) (layer F.Cu) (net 8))
 (segment (start 150.08 104.543) (end 151.1303 104.543) (width 0.25) (layer F.Cu) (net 8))
 (segment (start 150.691 108.56) (end 151.2163 108.56) (width 0.25) (layer F.Cu) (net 9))
 (segment (start 150.08 103.893) (end 151.1303 103.893) (width 0.25) (layer F.Cu) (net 9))
 (segment (start 151.5945 104.3572) (end 151.1303 103.893) (width 0.25) (layer F.Cu) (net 9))
 (segment (start 151.5945 108.1818) (end 151.5945 104.3572) (width 0.25) (layer F.Cu) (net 9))
 (segment (start 151.2163 108.56) (end 151.5945 108.1818) (width 0.25) (layer F.Cu) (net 9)))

